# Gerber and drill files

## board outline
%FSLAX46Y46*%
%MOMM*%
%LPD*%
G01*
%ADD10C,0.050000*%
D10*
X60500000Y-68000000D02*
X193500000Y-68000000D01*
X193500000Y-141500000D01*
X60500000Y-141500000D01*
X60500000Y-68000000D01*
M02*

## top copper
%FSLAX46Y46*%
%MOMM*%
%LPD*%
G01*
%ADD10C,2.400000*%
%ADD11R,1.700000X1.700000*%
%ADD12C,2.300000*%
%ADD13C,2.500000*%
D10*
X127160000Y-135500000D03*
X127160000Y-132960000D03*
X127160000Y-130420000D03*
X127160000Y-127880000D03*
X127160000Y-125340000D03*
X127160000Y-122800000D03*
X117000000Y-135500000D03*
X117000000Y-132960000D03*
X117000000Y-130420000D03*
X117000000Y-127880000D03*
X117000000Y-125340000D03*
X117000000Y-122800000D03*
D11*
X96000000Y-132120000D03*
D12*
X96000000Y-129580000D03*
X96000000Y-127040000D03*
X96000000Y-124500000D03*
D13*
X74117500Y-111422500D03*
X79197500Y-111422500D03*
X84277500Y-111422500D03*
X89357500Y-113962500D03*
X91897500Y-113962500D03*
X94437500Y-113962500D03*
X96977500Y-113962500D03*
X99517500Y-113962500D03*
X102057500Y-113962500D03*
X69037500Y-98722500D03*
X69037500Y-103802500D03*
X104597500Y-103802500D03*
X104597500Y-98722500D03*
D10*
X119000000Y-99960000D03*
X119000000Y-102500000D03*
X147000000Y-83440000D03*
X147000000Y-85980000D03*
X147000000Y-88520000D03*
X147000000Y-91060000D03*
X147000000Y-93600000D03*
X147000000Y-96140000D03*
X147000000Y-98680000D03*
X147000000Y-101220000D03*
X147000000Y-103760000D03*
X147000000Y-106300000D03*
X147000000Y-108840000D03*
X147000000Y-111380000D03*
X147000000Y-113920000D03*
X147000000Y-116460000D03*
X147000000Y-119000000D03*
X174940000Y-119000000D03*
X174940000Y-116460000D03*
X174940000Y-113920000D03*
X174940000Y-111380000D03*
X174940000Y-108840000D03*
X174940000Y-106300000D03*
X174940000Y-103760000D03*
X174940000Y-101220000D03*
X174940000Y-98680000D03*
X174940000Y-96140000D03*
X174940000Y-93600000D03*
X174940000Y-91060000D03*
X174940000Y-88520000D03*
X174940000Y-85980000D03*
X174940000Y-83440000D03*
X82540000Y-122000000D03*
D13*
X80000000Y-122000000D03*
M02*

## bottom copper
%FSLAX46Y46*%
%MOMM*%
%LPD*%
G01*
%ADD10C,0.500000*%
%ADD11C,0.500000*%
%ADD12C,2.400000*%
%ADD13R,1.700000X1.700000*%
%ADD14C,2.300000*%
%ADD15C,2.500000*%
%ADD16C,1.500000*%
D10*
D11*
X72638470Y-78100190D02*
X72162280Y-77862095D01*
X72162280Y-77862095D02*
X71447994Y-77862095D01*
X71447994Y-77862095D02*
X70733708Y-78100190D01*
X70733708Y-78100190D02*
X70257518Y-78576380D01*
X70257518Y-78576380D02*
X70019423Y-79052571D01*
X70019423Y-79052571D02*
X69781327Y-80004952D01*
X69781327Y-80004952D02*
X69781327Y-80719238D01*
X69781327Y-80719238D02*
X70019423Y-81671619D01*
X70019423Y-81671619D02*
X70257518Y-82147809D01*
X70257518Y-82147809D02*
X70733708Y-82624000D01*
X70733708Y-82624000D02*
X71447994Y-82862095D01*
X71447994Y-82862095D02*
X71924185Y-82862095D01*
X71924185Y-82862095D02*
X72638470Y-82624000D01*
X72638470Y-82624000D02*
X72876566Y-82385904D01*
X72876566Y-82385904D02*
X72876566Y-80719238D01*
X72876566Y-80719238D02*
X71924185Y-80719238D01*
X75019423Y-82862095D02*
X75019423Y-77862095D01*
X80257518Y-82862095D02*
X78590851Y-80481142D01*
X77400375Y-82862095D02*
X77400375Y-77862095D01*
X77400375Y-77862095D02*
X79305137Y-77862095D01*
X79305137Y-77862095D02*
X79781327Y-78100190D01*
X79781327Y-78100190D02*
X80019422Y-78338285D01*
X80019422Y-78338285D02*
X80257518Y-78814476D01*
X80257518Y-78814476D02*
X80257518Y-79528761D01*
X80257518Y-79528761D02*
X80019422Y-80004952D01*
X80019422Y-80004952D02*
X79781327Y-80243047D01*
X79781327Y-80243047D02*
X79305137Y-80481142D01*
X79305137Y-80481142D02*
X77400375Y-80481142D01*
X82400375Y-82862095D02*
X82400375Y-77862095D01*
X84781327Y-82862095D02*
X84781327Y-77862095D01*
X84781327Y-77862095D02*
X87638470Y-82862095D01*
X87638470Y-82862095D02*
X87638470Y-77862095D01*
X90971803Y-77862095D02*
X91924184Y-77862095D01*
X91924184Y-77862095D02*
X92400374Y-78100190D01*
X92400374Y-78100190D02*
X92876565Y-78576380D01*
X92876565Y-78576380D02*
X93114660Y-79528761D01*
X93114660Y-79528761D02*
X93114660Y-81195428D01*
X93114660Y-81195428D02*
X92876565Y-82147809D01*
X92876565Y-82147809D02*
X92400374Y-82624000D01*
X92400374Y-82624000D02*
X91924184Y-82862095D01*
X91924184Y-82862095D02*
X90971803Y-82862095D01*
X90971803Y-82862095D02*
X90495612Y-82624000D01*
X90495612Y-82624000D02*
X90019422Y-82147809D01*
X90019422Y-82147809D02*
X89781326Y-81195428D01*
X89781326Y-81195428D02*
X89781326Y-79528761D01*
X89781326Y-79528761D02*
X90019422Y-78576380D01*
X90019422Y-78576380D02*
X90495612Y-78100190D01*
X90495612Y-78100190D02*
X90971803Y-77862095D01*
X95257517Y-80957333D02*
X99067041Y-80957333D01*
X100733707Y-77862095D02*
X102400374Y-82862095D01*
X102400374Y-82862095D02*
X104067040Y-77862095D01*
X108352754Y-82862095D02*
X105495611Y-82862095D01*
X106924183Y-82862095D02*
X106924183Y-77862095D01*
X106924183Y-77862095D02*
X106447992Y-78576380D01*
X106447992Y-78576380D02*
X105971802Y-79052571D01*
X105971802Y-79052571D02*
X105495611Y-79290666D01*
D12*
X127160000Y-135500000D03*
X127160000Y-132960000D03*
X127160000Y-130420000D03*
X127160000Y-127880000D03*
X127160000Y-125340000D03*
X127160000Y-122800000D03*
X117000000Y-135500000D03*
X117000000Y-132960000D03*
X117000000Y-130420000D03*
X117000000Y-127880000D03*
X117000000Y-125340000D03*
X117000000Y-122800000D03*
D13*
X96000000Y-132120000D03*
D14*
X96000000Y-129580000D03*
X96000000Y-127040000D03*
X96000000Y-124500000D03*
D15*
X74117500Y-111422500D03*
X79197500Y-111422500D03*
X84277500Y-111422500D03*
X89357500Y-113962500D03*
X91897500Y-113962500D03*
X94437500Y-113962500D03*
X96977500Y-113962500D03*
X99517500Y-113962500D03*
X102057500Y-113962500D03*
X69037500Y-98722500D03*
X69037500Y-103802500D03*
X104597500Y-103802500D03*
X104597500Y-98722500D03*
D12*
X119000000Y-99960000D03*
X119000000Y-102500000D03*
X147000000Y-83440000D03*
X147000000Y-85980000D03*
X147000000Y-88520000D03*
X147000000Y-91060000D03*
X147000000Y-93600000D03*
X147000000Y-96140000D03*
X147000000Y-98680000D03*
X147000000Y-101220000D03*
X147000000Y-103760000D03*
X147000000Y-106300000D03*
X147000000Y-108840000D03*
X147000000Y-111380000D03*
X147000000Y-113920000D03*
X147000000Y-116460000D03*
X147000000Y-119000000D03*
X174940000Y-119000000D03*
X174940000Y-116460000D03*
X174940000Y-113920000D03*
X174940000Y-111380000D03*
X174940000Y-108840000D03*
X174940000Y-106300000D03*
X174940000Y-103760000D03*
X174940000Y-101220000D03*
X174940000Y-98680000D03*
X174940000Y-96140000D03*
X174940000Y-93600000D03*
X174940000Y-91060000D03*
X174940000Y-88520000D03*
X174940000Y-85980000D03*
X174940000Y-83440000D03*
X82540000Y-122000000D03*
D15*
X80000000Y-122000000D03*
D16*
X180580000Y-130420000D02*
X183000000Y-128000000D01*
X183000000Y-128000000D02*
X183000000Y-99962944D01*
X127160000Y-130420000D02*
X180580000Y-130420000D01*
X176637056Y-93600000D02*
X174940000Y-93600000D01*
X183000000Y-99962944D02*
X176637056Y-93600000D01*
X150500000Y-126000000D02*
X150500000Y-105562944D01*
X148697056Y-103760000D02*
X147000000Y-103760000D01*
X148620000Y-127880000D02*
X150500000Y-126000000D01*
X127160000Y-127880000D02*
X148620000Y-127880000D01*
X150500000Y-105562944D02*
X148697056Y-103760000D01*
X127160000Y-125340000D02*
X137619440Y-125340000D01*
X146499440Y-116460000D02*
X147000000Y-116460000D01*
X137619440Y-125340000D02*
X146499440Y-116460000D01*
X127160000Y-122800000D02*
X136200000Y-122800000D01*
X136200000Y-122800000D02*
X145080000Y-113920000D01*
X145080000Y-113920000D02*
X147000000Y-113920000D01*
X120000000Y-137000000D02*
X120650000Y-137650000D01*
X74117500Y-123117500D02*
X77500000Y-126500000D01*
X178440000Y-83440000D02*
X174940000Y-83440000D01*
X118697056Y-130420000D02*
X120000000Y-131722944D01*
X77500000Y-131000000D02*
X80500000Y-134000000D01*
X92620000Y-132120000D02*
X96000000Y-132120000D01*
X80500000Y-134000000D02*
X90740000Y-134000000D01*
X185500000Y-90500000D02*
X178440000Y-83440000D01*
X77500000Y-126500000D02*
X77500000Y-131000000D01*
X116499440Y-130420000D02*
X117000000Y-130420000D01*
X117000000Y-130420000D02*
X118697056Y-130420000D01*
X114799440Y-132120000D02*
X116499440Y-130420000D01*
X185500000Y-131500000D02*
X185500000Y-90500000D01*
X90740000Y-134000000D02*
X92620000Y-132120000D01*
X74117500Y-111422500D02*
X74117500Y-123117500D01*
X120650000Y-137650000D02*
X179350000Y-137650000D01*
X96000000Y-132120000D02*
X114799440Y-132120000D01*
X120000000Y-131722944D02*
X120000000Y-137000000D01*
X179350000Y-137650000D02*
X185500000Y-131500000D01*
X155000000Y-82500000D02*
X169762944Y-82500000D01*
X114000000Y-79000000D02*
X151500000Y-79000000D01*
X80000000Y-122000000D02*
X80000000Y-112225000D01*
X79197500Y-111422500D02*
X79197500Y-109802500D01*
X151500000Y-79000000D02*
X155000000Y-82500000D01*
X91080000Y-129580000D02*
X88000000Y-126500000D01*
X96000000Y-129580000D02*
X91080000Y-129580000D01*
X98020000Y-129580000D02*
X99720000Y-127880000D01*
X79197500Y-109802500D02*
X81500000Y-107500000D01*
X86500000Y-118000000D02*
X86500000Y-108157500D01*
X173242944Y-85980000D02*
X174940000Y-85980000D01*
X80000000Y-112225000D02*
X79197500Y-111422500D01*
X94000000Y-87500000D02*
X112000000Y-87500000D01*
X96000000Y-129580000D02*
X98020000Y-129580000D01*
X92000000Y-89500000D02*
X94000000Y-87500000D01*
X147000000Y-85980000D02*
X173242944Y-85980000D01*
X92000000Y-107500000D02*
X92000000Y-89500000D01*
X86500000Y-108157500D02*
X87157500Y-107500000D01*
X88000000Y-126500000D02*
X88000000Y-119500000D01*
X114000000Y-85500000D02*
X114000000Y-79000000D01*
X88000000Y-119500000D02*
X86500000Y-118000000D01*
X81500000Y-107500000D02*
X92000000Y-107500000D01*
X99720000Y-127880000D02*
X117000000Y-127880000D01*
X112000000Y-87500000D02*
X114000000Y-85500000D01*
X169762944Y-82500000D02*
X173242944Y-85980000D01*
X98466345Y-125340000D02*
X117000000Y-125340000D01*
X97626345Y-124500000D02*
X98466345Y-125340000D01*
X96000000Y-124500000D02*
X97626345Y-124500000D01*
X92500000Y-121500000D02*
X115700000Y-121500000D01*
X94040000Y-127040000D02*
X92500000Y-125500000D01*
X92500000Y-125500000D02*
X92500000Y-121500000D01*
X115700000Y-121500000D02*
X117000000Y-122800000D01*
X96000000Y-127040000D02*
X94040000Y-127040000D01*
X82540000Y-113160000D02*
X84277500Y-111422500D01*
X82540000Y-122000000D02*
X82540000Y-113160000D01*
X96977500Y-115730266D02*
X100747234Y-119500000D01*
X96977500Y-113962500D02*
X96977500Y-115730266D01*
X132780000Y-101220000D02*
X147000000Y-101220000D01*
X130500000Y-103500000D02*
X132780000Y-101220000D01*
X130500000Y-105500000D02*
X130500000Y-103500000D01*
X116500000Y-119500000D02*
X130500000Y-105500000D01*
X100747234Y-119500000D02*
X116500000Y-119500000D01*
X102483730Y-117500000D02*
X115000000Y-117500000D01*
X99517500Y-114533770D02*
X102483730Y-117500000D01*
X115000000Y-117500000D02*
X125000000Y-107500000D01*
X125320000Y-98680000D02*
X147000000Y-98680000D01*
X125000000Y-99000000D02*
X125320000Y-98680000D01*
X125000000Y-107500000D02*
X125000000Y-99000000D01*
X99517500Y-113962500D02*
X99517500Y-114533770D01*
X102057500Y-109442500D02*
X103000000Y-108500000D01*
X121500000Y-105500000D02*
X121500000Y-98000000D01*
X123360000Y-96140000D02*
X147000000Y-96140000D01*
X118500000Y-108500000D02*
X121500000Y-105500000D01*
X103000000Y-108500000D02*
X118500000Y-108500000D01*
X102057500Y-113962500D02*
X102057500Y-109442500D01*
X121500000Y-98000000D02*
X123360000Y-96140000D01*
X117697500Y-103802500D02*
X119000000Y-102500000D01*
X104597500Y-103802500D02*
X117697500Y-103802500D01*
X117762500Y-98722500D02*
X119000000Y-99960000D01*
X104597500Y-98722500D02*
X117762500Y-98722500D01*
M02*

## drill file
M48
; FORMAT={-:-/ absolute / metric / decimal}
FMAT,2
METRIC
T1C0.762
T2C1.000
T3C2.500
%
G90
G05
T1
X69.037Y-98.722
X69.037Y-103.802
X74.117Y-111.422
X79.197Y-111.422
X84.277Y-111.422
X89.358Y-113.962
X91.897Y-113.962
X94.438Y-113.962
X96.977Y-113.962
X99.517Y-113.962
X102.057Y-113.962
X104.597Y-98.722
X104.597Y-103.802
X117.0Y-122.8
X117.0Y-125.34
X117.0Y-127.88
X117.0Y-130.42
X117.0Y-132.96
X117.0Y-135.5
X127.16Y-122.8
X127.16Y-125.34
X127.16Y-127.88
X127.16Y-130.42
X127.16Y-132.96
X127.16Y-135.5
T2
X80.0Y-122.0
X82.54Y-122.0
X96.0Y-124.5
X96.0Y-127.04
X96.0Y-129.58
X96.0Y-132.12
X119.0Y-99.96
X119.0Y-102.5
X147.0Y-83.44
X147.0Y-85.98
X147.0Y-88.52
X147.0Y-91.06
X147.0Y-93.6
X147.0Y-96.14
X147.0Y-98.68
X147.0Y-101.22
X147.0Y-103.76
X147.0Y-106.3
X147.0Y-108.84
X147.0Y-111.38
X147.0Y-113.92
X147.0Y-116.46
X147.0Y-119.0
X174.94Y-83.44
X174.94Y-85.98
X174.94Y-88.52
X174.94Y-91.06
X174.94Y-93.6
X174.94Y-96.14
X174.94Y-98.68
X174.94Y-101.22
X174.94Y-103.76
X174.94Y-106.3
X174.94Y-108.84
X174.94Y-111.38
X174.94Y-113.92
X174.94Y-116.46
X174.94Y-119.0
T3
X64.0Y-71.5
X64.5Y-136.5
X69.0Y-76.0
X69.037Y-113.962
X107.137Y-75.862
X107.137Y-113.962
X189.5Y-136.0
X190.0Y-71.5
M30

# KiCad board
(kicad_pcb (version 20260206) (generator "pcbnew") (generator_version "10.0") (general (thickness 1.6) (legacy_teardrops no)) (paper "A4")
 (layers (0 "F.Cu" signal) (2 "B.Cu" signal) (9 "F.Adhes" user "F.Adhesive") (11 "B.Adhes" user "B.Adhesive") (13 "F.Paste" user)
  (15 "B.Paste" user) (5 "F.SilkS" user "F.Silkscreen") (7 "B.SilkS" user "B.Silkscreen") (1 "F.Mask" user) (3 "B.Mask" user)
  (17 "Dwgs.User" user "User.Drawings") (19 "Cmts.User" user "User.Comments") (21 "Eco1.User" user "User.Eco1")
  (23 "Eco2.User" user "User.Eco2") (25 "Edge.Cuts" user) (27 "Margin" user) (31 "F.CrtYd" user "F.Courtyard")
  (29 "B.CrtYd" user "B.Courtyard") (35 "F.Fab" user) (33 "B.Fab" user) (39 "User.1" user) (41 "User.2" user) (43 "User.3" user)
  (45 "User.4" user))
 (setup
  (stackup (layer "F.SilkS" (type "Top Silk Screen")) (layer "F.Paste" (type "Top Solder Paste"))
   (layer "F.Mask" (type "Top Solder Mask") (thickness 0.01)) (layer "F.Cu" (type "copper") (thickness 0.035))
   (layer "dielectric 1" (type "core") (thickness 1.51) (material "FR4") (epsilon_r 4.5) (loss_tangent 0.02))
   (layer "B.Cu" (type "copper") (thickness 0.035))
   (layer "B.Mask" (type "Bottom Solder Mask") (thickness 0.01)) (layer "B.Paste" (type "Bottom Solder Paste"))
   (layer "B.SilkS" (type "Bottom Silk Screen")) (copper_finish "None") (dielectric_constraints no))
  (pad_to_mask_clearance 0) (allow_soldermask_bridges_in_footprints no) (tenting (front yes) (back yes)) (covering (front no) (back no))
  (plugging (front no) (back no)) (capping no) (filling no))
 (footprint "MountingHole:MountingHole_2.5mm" (layer "F.Cu") (at 189.5 136)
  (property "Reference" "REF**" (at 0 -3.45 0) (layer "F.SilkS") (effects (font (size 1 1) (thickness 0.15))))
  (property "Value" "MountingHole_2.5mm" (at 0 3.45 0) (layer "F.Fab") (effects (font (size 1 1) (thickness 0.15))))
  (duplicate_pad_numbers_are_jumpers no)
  (pad "" np_thru_hole circle (at 0 0) (size 2.5 2.5) (drill 2.5) (layers "*.Cu" "*.Mask")))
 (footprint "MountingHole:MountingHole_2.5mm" (layer "F.Cu") (at 190 71.5)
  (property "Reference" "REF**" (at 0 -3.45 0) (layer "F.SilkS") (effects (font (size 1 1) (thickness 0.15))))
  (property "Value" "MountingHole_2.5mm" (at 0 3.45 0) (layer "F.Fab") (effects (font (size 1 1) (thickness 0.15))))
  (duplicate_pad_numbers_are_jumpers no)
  (pad "" np_thru_hole circle (at 0 0) (size 2.5 2.5) (drill 2.5) (layers "*.Cu" "*.Mask")))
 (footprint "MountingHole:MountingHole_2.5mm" (layer "F.Cu") (at 107.1375 75.8625)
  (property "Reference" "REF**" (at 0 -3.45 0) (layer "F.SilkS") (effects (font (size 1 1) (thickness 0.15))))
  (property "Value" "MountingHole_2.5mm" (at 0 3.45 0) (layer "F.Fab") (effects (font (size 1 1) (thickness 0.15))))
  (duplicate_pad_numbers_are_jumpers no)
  (pad "" np_thru_hole circle (at 0 0) (size 2.5 2.5) (drill 2.5) (layers "*.Cu" "*.Mask")))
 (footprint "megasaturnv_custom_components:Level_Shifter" (layer "F.Cu") (at 122.08 127.88 180)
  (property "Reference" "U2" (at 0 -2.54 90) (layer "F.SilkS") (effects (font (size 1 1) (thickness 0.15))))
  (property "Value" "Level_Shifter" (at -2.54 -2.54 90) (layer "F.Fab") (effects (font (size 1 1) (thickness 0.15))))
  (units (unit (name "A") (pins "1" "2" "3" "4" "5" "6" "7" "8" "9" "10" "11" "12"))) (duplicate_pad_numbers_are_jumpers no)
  (pad "1" thru_hole circle (at -5.08 -7.62 180) (size 2.4 2.4) (drill 0.762) (layers "*.Cu" "*.Mask") (remove_unused_layers no)
   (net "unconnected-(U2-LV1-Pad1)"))
  (pad "2" thru_hole circle (at -5.08 -5.08 180) (size 2.4 2.4) (drill 0.762) (layers "*.Cu" "*.Mask") (remove_unused_layers no)
   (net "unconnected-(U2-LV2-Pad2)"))
  (pad "3" thru_hole circle (at -5.08 -2.54 180) (size 2.4 2.4) (drill 0.762) (layers "*.Cu" "*.Mask") (remove_unused_layers no)
   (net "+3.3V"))
  (pad "4" thru_hole circle (at -5.08 0 180) (size 2.4 2.4) (drill 0.762) (layers "*.Cu" "*.Mask") (remove_unused_layers no)
   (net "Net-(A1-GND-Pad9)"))
  (pad "5" thru_hole circle (at -5.08 2.54 180) (size 2.4 2.4) (drill 0.762) (layers "*.Cu" "*.Mask") (remove_unused_layers no)
   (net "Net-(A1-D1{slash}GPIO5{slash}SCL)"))
  (pad "6" thru_hole circle (at -5.08 5.08 180) (size 2.4 2.4) (drill 0.762) (layers "*.Cu" "*.Mask") (remove_unused_layers no)
   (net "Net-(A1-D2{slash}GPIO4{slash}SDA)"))
  (pad "7" thru_hole circle (at 5.08 -7.62 180) (size 2.4 2.4) (drill 0.762) (layers "*.Cu" "*.Mask") (remove_unused_layers no)
   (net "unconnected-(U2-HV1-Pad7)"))
  (pad "8" thru_hole circle (at 5.08 -5.08 180) (size 2.4 2.4) (drill 0.762) (layers "*.Cu" "*.Mask") (remove_unused_layers no)
   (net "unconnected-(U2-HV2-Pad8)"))
  (pad "9" thru_hole circle (at 5.08 -2.54 180) (size 2.4 2.4) (drill 0.762) (layers "*.Cu" "*.Mask") (remove_unused_layers no) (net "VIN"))
  (pad "10" thru_hole circle (at 5.08 0 180) (size 2.4 2.4) (drill 0.762) (layers "*.Cu" "*.Mask") (remove_unused_layers no)
   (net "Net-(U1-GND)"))
  (pad "11" thru_hole circle (at 5.08 2.54 180) (size 2.4 2.4) (drill 0.762) (layers "*.Cu" "*.Mask") (remove_unused_layers no)
   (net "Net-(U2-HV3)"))
  (pad "12" thru_hole circle (at 5.08 5.08 180) (size 2.4 2.4) (drill 0.762) (layers "*.Cu" "*.Mask") (remove_unused_layers no)
   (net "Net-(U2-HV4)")))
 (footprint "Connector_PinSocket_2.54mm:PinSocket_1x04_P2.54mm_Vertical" (layer "F.Cu") (at 96 132.12 180)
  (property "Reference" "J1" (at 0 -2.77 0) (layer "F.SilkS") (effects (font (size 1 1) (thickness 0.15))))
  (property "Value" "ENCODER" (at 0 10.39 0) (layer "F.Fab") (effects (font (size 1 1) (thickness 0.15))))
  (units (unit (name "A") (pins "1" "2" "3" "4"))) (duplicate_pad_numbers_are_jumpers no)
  (pad "1" thru_hole rect (at 0 0 180) (size 1.7 1.7) (drill 1) (layers "*.Cu" "*.Mask") (remove_unused_layers no) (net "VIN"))
  (pad "2" thru_hole circle (at 0 2.54 180) (size 2.3 2.3) (drill 1) (layers "*.Cu" "*.Mask") (remove_unused_layers no) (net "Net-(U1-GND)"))
  (pad "3" thru_hole circle (at 0 5.08 180) (size 2.3 2.3) (drill 1) (layers "*.Cu" "*.Mask") (remove_unused_layers no) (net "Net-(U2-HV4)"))
  (pad "4" thru_hole circle (at 0 7.62 180) (size 2.3 2.3) (drill 1) (layers "*.Cu" "*.Mask") (remove_unused_layers no) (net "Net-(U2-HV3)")))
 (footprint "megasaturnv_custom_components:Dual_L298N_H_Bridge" (layer "F.Cu") (at 66.4975 116.5025)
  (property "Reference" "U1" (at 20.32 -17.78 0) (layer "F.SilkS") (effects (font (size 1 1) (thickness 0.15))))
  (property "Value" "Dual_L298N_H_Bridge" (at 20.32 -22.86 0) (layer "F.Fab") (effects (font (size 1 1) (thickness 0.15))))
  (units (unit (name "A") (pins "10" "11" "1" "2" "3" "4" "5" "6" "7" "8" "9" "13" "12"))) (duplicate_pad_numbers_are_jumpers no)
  (pad "1" thru_hole circle (at 7.62 -5.08) (size 2.5 2.5) (drill 0.762) (layers "*.Cu" "*.Mask") (remove_unused_layers no) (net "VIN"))
  (pad "2" thru_hole circle (at 12.7 -5.08) (size 2.5 2.5) (drill 0.762) (layers "*.Cu" "*.Mask") (remove_unused_layers no)
   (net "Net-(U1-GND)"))
  (pad "3" thru_hole circle (at 17.78 -5.08) (size 2.5 2.5) (drill 0.762) (layers "*.Cu" "*.Mask") (remove_unused_layers no)
   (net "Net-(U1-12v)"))
  (pad "4" thru_hole circle (at 22.86 -2.54) (size 2.5 2.5) (drill 0.762) (layers "*.Cu" "*.Mask") (remove_unused_layers no)
   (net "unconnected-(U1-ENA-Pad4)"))
  (pad "5" thru_hole circle (at 25.4 -2.54) (size 2.5 2.5) (drill 0.762) (layers "*.Cu" "*.Mask") (remove_unused_layers no)
   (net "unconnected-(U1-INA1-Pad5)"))
  (pad "6" thru_hole circle (at 27.94 -2.54) (size 2.5 2.5) (drill 0.762) (layers "*.Cu" "*.Mask") (remove_unused_layers no)
   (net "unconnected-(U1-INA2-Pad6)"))
  (pad "7" thru_hole circle (at 30.48 -2.54) (size 2.5 2.5) (drill 0.762) (layers "*.Cu" "*.Mask") (remove_unused_layers no)
   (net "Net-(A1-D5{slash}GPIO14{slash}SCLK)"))
  (pad "8" thru_hole circle (at 33.02 -2.54) (size 2.5 2.5) (drill 0.762) (layers "*.Cu" "*.Mask") (remove_unused_layers no)
   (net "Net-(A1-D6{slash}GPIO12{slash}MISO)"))
  (pad "9" thru_hole circle (at 35.56 -2.54) (size 2.5 2.5) (drill 0.762) (layers "*.Cu" "*.Mask") (remove_unused_layers no)
   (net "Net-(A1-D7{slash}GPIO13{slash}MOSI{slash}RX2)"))
  (pad "10" thru_hole circle (at 2.54 -17.78) (size 2.5 2.5) (drill 0.762) (layers "*.Cu" "*.Mask") (remove_unused_layers no)
   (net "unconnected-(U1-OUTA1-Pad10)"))
  (pad "11" thru_hole circle (at 2.54 -12.7) (size 2.5 2.5) (drill 0.762) (layers "*.Cu" "*.Mask") (remove_unused_layers no)
   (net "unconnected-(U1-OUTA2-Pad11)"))
  (pad "12" thru_hole circle (at 38.1 -12.7) (size 2.5 2.5) (drill 0.762) (layers "*.Cu" "*.Mask") (remove_unused_layers no)
   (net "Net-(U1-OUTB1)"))
  (pad "13" thru_hole circle (at 38.1 -17.78) (size 2.5 2.5) (drill 0.762) (layers "*.Cu" "*.Mask") (remove_unused_layers no)
   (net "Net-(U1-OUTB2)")))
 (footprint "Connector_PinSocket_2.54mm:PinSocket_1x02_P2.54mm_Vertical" (layer "F.Cu") (at 119 99.96)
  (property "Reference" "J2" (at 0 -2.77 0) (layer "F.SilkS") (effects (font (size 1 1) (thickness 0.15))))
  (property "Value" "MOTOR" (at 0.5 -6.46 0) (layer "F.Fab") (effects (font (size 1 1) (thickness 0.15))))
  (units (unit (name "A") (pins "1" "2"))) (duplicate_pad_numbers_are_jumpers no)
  (pad "1" thru_hole circle (at 0 0) (size 2.4 2.4) (drill 1) (layers "*.Cu" "*.Mask") (remove_unused_layers no) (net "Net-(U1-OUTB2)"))
  (pad "2" thru_hole circle (at 0 2.54) (size 2.4 2.4) (drill 1) (layers "*.Cu" "*.Mask") (remove_unused_layers no) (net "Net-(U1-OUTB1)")))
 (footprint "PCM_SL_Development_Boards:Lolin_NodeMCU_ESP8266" (layer "F.Cu") (at 160.97 101.22)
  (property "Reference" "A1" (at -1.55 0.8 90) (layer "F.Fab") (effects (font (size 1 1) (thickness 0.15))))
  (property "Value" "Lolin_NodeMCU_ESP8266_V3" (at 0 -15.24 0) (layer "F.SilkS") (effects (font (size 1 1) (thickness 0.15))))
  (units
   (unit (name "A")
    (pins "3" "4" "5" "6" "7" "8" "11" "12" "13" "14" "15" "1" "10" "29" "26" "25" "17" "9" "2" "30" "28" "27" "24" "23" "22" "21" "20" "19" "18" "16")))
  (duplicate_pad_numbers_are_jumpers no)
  (pad "1" thru_hole circle (at -13.97 -17.78 270) (size 2.4 2.4) (drill 1) (layers "*.Cu" "*.Mask") (remove_unused_layers no)
   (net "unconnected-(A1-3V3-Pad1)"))
  (pad "2" thru_hole circle (at -13.97 -15.24 270) (size 2.4 2.4) (drill 1) (layers "*.Cu" "*.Mask") (remove_unused_layers no)
   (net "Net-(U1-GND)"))
  (pad "3" thru_hole circle (at -13.97 -12.7 270) (size 2.4 2.4) (drill 1) (layers "*.Cu" "*.Mask") (remove_unused_layers no)
   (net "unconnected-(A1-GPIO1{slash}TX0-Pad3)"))
  (pad "4" thru_hole circle (at -13.97 -10.16 270) (size 2.4 2.4) (drill 1) (layers "*.Cu" "*.Mask") (remove_unused_layers no)
   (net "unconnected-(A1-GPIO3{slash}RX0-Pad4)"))
  (pad "5" thru_hole circle (at -13.97 -7.62 270) (size 2.4 2.4) (drill 1) (layers "*.Cu" "*.Mask") (remove_unused_layers no)
   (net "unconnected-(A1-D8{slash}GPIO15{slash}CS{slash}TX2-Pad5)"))
  (pad "6" thru_hole circle (at -13.97 -5.08 270) (size 2.4 2.4) (drill 1) (layers "*.Cu" "*.Mask") (remove_unused_layers no)
   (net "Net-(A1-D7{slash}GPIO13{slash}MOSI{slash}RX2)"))
  (pad "7" thru_hole circle (at -13.97 -2.54 270) (size 2.4 2.4) (drill 1) (layers "*.Cu" "*.Mask") (remove_unused_layers no)
   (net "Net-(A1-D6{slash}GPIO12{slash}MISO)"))
  (pad "8" thru_hole circle (at -13.97 0 270) (size 2.4 2.4) (drill 1) (layers "*.Cu" "*.Mask") (remove_unused_layers no)
   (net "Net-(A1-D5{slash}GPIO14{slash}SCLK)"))
  (pad "9" thru_hole circle (at -13.97 2.54 270) (size 2.4 2.4) (drill 1) (layers "*.Cu" "*.Mask") (remove_unused_layers no)
   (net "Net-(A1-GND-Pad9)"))
  (pad "10" thru_hole circle (at -13.97 5.08 270) (size 2.4 2.4) (drill 1) (layers "*.Cu" "*.Mask") (remove_unused_layers no)
   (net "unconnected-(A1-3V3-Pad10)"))
  (pad "11" thru_hole circle (at -13.97 7.62 270) (size 2.4 2.4) (drill 1) (layers "*.Cu" "*.Mask") (remove_unused_layers no)
   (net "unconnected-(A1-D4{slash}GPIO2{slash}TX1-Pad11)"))
  (pad "12" thru_hole circle (at -13.97 10.16 270) (size 2.4 2.4) (drill 1) (layers "*.Cu" "*.Mask") (remove_unused_layers no)
   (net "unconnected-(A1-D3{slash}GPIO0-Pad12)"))
  (pad "13" thru_hole circle (at -13.97 12.7 270) (size 2.4 2.4) (drill 1) (layers "*.Cu" "*.Mask") (remove_unused_layers no)
   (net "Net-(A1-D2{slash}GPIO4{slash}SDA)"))
  (pad "14" thru_hole circle (at -13.97 15.24 270) (size 2.4 2.4) (drill 1) (layers "*.Cu" "*.Mask") (remove_unused_layers no)
   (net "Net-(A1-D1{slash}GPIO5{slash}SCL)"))
  (pad "15" thru_hole circle (at -13.97 17.78 270) (size 2.4 2.4) (drill 1) (layers "*.Cu" "*.Mask") (remove_unused_layers no)
   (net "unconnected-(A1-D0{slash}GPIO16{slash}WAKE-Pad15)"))
  (pad "16" thru_hole circle (at 13.97 17.78 270) (size 2.4 2.4) (drill 1) (layers "*.Cu" "*.Mask") (remove_unused_layers no)
   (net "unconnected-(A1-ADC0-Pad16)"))
  (pad "17" thru_hole circle (at 13.97 15.24 270) (size 2.4 2.4) (drill 1) (layers "*.Cu" "*.Mask") (remove_unused_layers no)
   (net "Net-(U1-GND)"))
  (pad "18" thru_hole circle (at 13.97 12.7 270) (size 2.4 2.4) (drill 1) (layers "*.Cu" "*.Mask") (remove_unused_layers no)
   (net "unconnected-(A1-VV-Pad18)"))
  (pad "19" thru_hole circle (at 13.97 10.16 270) (size 2.4 2.4) (drill 1) (layers "*.Cu" "*.Mask") (remove_unused_layers no)
   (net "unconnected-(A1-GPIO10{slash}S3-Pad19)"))
  (pad "20" thru_hole circle (at 13.97 7.62 270) (size 2.4 2.4) (drill 1) (layers "*.Cu" "*.Mask") (remove_unused_layers no)
   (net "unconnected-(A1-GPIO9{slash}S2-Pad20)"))
  (pad "21" thru_hole circle (at 13.97 5.08 270) (size 2.4 2.4) (drill 1) (layers "*.Cu" "*.Mask") (remove_unused_layers no)
   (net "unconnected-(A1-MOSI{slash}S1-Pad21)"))
  (pad "22" thru_hole circle (at 13.97 2.54 270) (size 2.4 2.4) (drill 1) (layers "*.Cu" "*.Mask") (remove_unused_layers no)
   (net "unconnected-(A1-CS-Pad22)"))
  (pad "23" thru_hole circle (at 13.97 0 270) (size 2.4 2.4) (drill 1) (layers "*.Cu" "*.Mask") (remove_unused_layers no)
   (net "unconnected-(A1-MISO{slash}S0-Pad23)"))
  (pad "24" thru_hole circle (at 13.97 -2.54 270) (size 2.4 2.4) (drill 1) (layers "*.Cu" "*.Mask") (remove_unused_layers no)
   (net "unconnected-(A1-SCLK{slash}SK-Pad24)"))
  (pad "25" thru_hole circle (at 13.97 -5.08 270) (size 2.4 2.4) (drill 1) (layers "*.Cu" "*.Mask") (remove_unused_layers no)
   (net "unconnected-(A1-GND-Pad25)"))
  (pad "26" thru_hole circle (at 13.97 -7.62 270) (size 2.4 2.4) (drill 1) (layers "*.Cu" "*.Mask") (remove_unused_layers no) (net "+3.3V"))
  (pad "27" thru_hole circle (at 13.97 -10.16 270) (size 2.4 2.4) (drill 1) (layers "*.Cu" "*.Mask") (remove_unused_layers no)
   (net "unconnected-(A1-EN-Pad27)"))
  (pad "28" thru_hole circle (at 13.97 -12.7 270) (size 2.4 2.4) (drill 1) (layers "*.Cu" "*.Mask") (remove_unused_layers no)
   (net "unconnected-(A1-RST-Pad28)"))
  (pad "29" thru_hole circle (at 13.97 -15.24 270) (size 2.4 2.4) (drill 1) (layers "*.Cu" "*.Mask") (remove_unused_layers no)
   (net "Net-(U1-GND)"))
  (pad "30" thru_hole circle (at 13.97 -17.78 270) (size 2.4 2.4) (drill 1) (layers "*.Cu" "*.Mask") (remove_unused_layers no) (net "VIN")))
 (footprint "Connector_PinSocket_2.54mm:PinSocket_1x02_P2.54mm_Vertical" (layer "F.Cu") (at 82.54 122 -90)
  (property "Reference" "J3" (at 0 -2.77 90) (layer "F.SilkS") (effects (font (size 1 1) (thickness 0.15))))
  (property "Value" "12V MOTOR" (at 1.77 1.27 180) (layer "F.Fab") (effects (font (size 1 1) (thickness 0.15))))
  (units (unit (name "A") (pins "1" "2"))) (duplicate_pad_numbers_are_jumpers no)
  (pad "1" thru_hole circle (at 0 0 270) (size 2.4 2.4) (drill 1) (layers "*.Cu" "*.Mask") (remove_unused_layers no) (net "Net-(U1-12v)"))
  (pad "2" thru_hole circle (at 0 2.54 270) (size 2.5 2.5) (drill 1) (layers "*.Cu" "*.Mask") (remove_unused_layers no) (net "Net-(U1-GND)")))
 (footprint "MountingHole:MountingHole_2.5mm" (layer "F.Cu") (at 64 71.5)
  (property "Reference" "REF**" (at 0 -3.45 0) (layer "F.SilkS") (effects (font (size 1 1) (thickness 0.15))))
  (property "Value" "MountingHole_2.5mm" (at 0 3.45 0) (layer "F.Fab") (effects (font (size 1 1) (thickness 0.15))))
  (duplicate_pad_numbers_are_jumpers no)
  (pad "" np_thru_hole circle (at 0 0) (size 2.5 2.5) (drill 2.5) (layers "*.Cu" "*.Mask")))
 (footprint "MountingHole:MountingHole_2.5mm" (layer "F.Cu") (at 69 76)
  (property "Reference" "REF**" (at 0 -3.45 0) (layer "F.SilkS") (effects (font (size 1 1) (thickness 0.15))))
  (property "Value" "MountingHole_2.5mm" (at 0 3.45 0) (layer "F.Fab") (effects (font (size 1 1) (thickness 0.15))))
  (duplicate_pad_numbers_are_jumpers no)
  (pad "" np_thru_hole circle (at 0 0) (size 2.5 2.5) (drill 2.5) (layers "*.Cu" "*.Mask")))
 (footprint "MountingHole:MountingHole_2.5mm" (layer "F.Cu") (at 64.5 136.5)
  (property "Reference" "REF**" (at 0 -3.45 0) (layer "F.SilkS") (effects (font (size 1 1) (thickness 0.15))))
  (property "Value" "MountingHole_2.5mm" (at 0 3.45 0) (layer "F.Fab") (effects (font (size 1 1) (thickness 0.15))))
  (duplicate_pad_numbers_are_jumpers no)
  (pad "" np_thru_hole circle (at 0 0) (size 2.5 2.5) (drill 2.5) (layers "*.Cu" "*.Mask")))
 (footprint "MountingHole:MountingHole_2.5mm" (layer "F.Cu") (at 107.1375 113.9625)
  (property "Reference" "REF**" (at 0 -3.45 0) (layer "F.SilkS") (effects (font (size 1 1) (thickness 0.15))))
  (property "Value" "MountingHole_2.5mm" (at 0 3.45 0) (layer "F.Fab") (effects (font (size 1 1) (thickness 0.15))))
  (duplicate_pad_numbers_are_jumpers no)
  (pad "" np_thru_hole circle (at 0 0) (size 2.5 2.5) (drill 2.5) (layers "*.Cu" "*.Mask")))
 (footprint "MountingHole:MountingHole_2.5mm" (layer "F.Cu") (at 69.0375 113.9625)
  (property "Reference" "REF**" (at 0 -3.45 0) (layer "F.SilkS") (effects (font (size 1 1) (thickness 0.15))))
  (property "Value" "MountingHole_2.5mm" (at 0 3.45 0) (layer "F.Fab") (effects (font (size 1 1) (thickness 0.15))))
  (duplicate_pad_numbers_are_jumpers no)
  (pad "" np_thru_hole circle (at 0 0) (size 2.5 2.5) (drill 2.5) (layers "*.Cu" "*.Mask")))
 (gr_rect (start 60.5 68) (end 193.5 141.5) (stroke (width 0.05) (type default)) (fill no) (layer "Edge.Cuts"))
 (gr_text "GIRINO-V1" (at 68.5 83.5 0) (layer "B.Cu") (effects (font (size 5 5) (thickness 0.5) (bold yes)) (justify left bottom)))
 (segment (start 180.58 130.42) (end 183 128) (width 1.5) (layer "B.Cu") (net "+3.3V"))
 (segment (start 183 128) (end 183 99.962944) (width 1.5) (layer "B.Cu") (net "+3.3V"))
 (segment (start 127.16 130.42) (end 180.58 130.42) (width 1.5) (layer "B.Cu") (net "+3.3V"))
 (segment (start 176.637056 93.6) (end 174.94 93.6) (width 1.5) (layer "B.Cu") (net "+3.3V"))
 (segment (start 183 99.962944) (end 176.637056 93.6) (width 1.5) (layer "B.Cu") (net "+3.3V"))
 (segment (start 150.5 126) (end 150.5 105.562944) (width 1.5) (layer "B.Cu") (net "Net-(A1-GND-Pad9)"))
 (segment (start 148.697056 103.76) (end 147 103.76) (width 1.5) (layer "B.Cu") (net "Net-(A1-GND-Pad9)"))
 (segment (start 148.62 127.88) (end 150.5 126) (width 1.5) (layer "B.Cu") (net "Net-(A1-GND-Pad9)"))
 (segment (start 127.16 127.88) (end 148.62 127.88) (width 1.5) (layer "B.Cu") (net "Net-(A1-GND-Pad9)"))
 (segment (start 150.5 105.562944) (end 148.697056 103.76) (width 1.5) (layer "B.Cu") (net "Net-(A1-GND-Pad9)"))
 (segment (start 127.16 125.34) (end 137.61944 125.34) (width 1.5) (layer "B.Cu") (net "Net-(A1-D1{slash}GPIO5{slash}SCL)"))
 (segment (start 146.49944 116.46) (end 147 116.46) (width 1.5) (layer "B.Cu") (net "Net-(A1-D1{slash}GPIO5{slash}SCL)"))
 (segment (start 137.61944 125.34) (end 146.49944 116.46) (width 1.5) (layer "B.Cu") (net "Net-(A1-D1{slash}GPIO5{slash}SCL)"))
 (segment (start 127.16 122.8) (end 136.2 122.8) (width 1.5) (layer "B.Cu") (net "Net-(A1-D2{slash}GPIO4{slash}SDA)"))
 (segment (start 136.2 122.8) (end 145.08 113.92) (width 1.5) (layer "B.Cu") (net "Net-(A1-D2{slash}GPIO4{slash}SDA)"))
 (segment (start 145.08 113.92) (end 147 113.92) (width 1.5) (layer "B.Cu") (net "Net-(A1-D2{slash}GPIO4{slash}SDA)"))
 (segment (start 120 137) (end 120.65 137.65) (width 1.5) (layer "B.Cu") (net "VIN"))
 (segment (start 74.1175 123.1175) (end 77.5 126.5) (width 1.5) (layer "B.Cu") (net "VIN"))
 (segment (start 178.44 83.44) (end 174.94 83.44) (width 1.5) (layer "B.Cu") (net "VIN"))
 (segment (start 118.697056 130.42) (end 120 131.722944) (width 1.5) (layer "B.Cu") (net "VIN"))
 (segment (start 77.5 131) (end 80.5 134) (width 1.5) (layer "B.Cu") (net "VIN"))
 (segment (start 92.62 132.12) (end 96 132.12) (width 1.5) (layer "B.Cu") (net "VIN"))
 (segment (start 80.5 134) (end 90.74 134) (width 1.5) (layer "B.Cu") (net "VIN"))
 (segment (start 185.5 90.5) (end 178.44 83.44) (width 1.5) (layer "B.Cu") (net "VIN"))
 (segment (start 77.5 126.5) (end 77.5 131) (width 1.5) (layer "B.Cu") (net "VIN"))
 (segment (start 116.49944 130.42) (end 117 130.42) (width 1.5) (layer "B.Cu") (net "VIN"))
 (segment (start 117 130.42) (end 118.697056 130.42) (width 1.5) (layer "B.Cu") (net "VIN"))
 (segment (start 114.79944 132.12) (end 116.49944 130.42) (width 1.5) (layer "B.Cu") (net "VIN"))
 (segment (start 185.5 131.5) (end 185.5 90.5) (width 1.5) (layer "B.Cu") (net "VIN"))
 (segment (start 90.74 134) (end 92.62 132.12) (width 1.5) (layer "B.Cu") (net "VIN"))
 (segment (start 74.1175 111.4225) (end 74.1175 123.1175) (width 1.5) (layer "B.Cu") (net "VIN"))
 (segment (start 120.65 137.65) (end 179.35 137.65) (width 1.5) (layer "B.Cu") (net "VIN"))
 (segment (start 96 132.12) (end 114.79944 132.12) (width 1.5) (layer "B.Cu") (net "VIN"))
 (segment (start 120 131.722944) (end 120 137) (width 1.5) (layer "B.Cu") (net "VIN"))
 (segment (start 179.35 137.65) (end 185.5 131.5) (width 1.5) (layer "B.Cu") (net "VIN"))
 (segment (start 155 82.5) (end 169.762944 82.5) (width 1.5) (layer "B.Cu") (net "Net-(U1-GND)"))
 (segment (start 114 79) (end 151.5 79) (width 1.5) (layer "B.Cu") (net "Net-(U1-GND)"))
 (segment (start 80 122) (end 80 112.225) (width 1.5) (layer "B.Cu") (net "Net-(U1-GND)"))
 (segment (start 79.1975 111.4225) (end 79.1975 109.8025) (width 1.5) (layer "B.Cu") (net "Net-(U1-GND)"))
 (segment (start 151.5 79) (end 155 82.5) (width 1.5) (layer "B.Cu") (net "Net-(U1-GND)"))
 (segment (start 91.08 129.58) (end 88 126.5) (width 1.5) (layer "B.Cu") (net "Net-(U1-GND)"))
 (segment (start 96 129.58) (end 91.08 129.58) (width 1.5) (layer "B.Cu") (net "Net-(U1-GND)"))
 (segment (start 98.02 129.58) (end 99.72 127.88) (width 1.5) (layer "B.Cu") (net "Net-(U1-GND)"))
 (segment (start 79.1975 109.8025) (end 81.5 107.5) (width 1.5) (layer "B.Cu") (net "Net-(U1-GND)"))
 (segment (start 86.5 118) (end 86.5 108.1575) (width 1.5) (layer "B.Cu") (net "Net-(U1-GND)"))
 (segment (start 173.242944 85.98) (end 174.94 85.98) (width 1.5) (layer "B.Cu") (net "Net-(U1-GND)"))
 (segment (start 80 112.225) (end 79.1975 111.4225) (width 1.5) (layer "B.Cu") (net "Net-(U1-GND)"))
 (segment (start 94 87.5) (end 112 87.5) (width 1.5) (layer "B.Cu") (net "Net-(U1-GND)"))
 (segment (start 96 129.58) (end 98.02 129.58) (width 1.5) (layer "B.Cu") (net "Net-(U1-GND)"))
 (segment (start 92 89.5) (end 94 87.5) (width 1.5) (layer "B.Cu") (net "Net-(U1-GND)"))
 (segment (start 147 85.98) (end 173.242944 85.98) (width 1.5) (layer "B.Cu") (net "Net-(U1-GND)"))
 (segment (start 92 107.5) (end 92 89.5) (width 1.5) (layer "B.Cu") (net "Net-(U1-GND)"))
 (segment (start 86.5 108.1575) (end 87.1575 107.5) (width 1.5) (layer "B.Cu") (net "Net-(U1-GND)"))
 (segment (start 88 126.5) (end 88 119.5) (width 1.5) (layer "B.Cu") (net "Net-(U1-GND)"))
 (segment (start 114 85.5) (end 114 79) (width 1.5) (layer "B.Cu") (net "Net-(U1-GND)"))
 (segment (start 88 119.5) (end 86.5 118) (width 1.5) (layer "B.Cu") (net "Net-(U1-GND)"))
 (segment (start 81.5 107.5) (end 92 107.5) (width 1.5) (layer "B.Cu") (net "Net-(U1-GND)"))
 (segment (start 99.72 127.88) (end 117 127.88) (width 1.5) (layer "B.Cu") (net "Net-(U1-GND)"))
 (segment (start 112 87.5) (end 114 85.5) (width 1.5) (layer "B.Cu") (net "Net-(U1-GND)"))
 (segment (start 169.762944 82.5) (end 173.242944 85.98) (width 1.5) (layer "B.Cu") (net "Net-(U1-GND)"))
 (segment (start 98.466345 125.34) (end 117 125.34) (width 1.5) (layer "B.Cu") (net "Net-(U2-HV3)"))
 (segment (start 97.626345 124.5) (end 98.466345 125.34) (width 1.5) (layer "B.Cu") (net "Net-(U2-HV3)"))
 (segment (start 96 124.5) (end 97.626345 124.5) (width 1.5) (layer "B.Cu") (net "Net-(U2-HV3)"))
 (segment (start 92.5 121.5) (end 115.7 121.5) (width 1.5) (layer "B.Cu") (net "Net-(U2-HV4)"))
 (segment (start 94.04 127.04) (end 92.5 125.5) (width 1.5) (layer "B.Cu") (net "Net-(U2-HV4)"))
 (segment (start 92.5 125.5) (end 92.5 121.5) (width 1.5) (layer "B.Cu") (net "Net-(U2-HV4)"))
 (segment (start 115.7 121.5) (end 117 122.8) (width 1.5) (layer "B.Cu") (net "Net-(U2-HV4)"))
 (segment (start 96 127.04) (end 94.04 127.04) (width 1.5) (layer "B.Cu") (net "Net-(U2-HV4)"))
 (segment (start 82.54 113.16) (end 84.2775 111.4225) (width 1.5) (layer "B.Cu") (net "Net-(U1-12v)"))
 (segment (start 82.54 122) (end 82.54 113.16) (width 1.5) (layer "B.Cu") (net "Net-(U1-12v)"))
 (segment (start 96.9775 115.730266) (end 100.747234 119.5) (width 1.5) (layer "B.Cu") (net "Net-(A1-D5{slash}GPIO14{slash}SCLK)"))
 (segment (start 96.9775 113.9625) (end 96.9775 115.730266) (width 1.5) (layer "B.Cu") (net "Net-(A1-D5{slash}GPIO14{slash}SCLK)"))
 (segment (start 132.78 101.22) (end 147 101.22) (width 1.5) (layer "B.Cu") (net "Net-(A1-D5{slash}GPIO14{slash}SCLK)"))
 (segment (start 130.5 103.5) (end 132.78 101.22) (width 1.5) (layer "B.Cu") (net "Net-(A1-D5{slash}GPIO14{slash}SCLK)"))
 (segment (start 130.5 105.5) (end 130.5 103.5) (width 1.5) (layer "B.Cu") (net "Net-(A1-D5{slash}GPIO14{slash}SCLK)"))
 (segment (start 116.5 119.5) (end 130.5 105.5) (width 1.5) (layer "B.Cu") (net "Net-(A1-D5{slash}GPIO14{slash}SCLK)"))
 (segment (start 100.747234 119.5) (end 116.5 119.5) (width 1.5) (layer "B.Cu") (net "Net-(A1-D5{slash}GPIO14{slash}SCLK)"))
 (segment (start 102.48373 117.5) (end 115 117.5) (width 1.5) (layer "B.Cu") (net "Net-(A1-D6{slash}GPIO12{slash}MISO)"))
 (segment (start 99.5175 114.53377) (end 102.48373 117.5) (width 1.5) (layer "B.Cu") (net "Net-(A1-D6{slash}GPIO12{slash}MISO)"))
 (segment (start 115 117.5) (end 125 107.5) (width 1.5) (layer "B.Cu") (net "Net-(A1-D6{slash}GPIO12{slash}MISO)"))
 (segment (start 125.32 98.68) (end 147 98.68) (width 1.5) (layer "B.Cu") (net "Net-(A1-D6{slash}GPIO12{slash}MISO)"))
 (segment (start 125 99) (end 125.32 98.68) (width 1.5) (layer "B.Cu") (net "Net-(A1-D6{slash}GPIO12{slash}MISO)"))
 (segment (start 125 107.5) (end 125 99) (width 1.5) (layer "B.Cu") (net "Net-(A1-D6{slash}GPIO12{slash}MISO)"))
 (segment (start 99.5175 113.9625) (end 99.5175 114.53377) (width 1.5) (layer "B.Cu") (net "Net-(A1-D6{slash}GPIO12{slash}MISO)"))
 (segment (start 102.0575 109.4425) (end 103 108.5) (width 1.5) (layer "B.Cu") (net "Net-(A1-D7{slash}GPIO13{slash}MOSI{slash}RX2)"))
 (segment (start 121.5 105.5) (end 121.5 98) (width 1.5) (layer "B.Cu") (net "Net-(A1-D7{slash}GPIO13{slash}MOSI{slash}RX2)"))
 (segment (start 123.36 96.14) (end 147 96.14) (width 1.5) (layer "B.Cu") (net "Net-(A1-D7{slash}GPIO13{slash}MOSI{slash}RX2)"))
 (segment (start 118.5 108.5) (end 121.5 105.5) (width 1.5) (layer "B.Cu") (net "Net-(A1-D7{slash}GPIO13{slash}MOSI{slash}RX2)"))
 (segment (start 103 108.5) (end 118.5 108.5) (width 1.5) (layer "B.Cu") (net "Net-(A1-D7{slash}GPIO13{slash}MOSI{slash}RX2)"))
 (segment (start 102.0575 113.9625) (end 102.0575 109.4425) (width 1.5) (layer "B.Cu") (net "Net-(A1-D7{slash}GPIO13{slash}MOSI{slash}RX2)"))
 (segment (start 121.5 98) (end 123.36 96.14) (width 1.5) (layer "B.Cu") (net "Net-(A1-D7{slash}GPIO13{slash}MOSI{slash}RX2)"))
 (segment (start 117.6975 103.8025) (end 119 102.5) (width 1.5) (layer "B.Cu") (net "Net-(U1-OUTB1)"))
 (segment (start 104.5975 103.8025) (end 117.6975 103.8025) (width 1.5) (layer "B.Cu") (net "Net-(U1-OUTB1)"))
 (segment (start 117.7625 98.7225) (end 119 99.96) (width 1.5) (layer "B.Cu") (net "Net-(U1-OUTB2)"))
 (segment (start 104.5975 98.7225) (end 117.7625 98.7225) (width 1.5) (layer "B.Cu") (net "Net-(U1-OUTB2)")))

